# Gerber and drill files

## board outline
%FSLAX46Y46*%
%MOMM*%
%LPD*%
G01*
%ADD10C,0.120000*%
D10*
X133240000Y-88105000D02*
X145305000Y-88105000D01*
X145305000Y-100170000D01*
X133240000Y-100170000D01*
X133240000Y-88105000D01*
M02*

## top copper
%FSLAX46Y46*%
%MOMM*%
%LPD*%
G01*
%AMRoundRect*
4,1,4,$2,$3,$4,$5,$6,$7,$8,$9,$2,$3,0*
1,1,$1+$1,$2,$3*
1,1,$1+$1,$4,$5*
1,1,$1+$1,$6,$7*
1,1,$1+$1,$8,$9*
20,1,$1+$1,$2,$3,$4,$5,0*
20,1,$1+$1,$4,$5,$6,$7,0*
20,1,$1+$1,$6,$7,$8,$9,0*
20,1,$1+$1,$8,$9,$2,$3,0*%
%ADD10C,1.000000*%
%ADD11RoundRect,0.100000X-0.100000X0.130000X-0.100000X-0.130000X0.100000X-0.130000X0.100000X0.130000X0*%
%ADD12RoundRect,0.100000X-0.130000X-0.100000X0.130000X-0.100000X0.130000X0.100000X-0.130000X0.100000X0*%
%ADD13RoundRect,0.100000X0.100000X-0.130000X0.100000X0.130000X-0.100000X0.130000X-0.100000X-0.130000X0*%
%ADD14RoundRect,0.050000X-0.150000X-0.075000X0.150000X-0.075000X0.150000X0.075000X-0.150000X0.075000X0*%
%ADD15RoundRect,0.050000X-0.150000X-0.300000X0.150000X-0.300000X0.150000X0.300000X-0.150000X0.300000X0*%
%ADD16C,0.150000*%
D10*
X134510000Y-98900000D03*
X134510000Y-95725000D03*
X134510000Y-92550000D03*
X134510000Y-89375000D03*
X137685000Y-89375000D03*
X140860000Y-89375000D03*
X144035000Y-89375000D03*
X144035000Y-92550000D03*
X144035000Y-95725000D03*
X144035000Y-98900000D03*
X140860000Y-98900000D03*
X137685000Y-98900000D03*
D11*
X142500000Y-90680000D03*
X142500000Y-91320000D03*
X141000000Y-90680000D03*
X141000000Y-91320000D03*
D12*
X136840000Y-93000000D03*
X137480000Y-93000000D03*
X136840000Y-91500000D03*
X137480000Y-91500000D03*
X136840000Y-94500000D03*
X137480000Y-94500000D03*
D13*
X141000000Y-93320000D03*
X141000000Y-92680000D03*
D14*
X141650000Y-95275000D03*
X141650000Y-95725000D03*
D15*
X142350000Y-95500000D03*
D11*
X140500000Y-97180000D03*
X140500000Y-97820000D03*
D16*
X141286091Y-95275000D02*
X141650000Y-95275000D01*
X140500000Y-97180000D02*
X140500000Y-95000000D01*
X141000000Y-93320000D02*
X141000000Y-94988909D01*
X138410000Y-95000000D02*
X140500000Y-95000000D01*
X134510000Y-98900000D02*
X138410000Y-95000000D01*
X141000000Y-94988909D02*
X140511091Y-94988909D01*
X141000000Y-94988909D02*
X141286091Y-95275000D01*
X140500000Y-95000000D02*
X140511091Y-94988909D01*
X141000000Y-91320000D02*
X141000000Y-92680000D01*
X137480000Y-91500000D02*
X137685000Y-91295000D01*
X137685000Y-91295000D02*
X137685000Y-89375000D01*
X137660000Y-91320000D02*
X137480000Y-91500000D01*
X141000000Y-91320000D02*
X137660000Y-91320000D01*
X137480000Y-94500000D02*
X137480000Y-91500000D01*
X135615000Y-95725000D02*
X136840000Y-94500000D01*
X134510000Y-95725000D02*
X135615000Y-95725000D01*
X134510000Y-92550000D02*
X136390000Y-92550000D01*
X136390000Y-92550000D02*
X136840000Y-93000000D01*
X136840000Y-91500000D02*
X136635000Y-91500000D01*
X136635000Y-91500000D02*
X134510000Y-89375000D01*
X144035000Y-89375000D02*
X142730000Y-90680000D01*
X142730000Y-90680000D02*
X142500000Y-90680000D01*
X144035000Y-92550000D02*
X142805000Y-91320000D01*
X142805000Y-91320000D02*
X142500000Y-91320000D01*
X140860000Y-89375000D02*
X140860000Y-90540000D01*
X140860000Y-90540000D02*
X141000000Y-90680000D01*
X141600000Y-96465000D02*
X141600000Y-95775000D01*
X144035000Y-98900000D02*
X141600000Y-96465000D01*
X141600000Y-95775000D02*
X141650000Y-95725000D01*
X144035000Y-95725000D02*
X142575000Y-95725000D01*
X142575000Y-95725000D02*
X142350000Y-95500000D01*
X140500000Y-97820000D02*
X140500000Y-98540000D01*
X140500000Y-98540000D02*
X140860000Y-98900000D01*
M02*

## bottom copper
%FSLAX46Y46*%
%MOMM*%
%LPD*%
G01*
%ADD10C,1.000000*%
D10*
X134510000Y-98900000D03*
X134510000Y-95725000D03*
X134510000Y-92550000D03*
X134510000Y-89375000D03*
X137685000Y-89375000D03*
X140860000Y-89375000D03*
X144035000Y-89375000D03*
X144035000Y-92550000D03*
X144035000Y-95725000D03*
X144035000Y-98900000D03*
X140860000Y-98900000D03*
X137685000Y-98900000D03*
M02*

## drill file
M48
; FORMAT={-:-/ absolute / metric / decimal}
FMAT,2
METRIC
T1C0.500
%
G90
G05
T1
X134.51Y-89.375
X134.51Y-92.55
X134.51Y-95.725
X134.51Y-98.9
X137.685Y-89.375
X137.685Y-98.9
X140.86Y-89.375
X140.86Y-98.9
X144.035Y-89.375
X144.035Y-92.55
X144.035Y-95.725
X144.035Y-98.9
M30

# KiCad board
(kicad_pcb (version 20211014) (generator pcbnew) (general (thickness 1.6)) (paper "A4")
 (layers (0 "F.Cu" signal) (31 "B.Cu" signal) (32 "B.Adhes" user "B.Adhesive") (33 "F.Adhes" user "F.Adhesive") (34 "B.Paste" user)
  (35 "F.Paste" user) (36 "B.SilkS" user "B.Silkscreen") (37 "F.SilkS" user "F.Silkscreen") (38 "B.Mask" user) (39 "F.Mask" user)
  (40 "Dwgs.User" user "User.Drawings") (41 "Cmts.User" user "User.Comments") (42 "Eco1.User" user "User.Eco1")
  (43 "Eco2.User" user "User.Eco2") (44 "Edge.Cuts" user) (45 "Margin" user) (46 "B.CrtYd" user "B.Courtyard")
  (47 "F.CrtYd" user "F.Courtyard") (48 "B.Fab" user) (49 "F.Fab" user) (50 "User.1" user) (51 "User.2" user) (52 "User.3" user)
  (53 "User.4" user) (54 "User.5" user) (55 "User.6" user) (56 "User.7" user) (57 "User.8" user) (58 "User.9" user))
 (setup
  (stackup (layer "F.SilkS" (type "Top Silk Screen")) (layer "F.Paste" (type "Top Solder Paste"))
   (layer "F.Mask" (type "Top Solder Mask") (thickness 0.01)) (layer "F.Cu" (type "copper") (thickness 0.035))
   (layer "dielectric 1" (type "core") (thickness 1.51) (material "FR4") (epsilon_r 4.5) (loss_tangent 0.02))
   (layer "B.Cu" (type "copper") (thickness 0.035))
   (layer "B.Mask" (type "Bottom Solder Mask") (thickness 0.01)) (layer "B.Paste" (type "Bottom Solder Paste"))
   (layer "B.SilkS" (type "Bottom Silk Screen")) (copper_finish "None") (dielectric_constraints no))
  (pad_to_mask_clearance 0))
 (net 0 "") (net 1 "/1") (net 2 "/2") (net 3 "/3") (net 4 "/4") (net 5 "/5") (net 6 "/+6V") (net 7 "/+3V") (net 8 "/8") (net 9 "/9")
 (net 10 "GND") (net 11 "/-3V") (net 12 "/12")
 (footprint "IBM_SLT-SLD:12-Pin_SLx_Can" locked (layer "F.Cu") (at 134.51 98.9)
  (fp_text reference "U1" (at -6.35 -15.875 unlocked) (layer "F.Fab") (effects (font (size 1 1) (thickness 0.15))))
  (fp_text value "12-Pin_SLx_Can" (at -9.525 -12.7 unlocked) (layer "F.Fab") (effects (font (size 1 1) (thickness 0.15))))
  (fp_rect (start -1.27 -10.795) (end 10.795 1.27) (layer "Edge.Cuts") (width 0.12) (fill none))
  (pad "1" thru_hole circle locked (at 0 0) (size 1 1) (drill 0.5) (layers *.Cu *.Mask) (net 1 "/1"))
  (pad "2" thru_hole circle locked (at 0 -3.175) (size 1 1) (drill 0.5) (layers *.Cu *.Mask) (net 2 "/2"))
  (pad "3" thru_hole circle locked (at 0 -6.35) (size 1 1) (drill 0.5) (layers *.Cu *.Mask) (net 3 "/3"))
  (pad "4" thru_hole circle locked (at 0 -9.525) (size 1 1) (drill 0.5) (layers *.Cu *.Mask) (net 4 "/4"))
  (pad "5" thru_hole circle locked (at 3.175 -9.525) (size 1 1) (drill 0.5) (layers *.Cu *.Mask) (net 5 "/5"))
  (pad "6" thru_hole circle locked (at 6.35 -9.525) (size 1 1) (drill 0.5) (layers *.Cu *.Mask) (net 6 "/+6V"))
  (pad "7" thru_hole circle locked (at 9.525 -9.525) (size 1 1) (drill 0.5) (layers *.Cu *.Mask) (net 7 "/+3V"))
  (pad "8" thru_hole circle locked (at 9.525 -6.35) (size 1 1) (drill 0.5) (layers *.Cu *.Mask) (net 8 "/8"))
  (pad "9" thru_hole circle locked (at 9.525 -3.175) (size 1 1) (drill 0.5) (layers *.Cu *.Mask) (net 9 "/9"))
  (pad "10" thru_hole circle locked (at 9.525 0) (size 1 1) (drill 0.5) (layers *.Cu *.Mask) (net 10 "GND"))
  (pad "11" thru_hole circle locked (at 6.35 0) (size 1 1) (drill 0.5) (layers *.Cu *.Mask) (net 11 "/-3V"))
  (pad "12" thru_hole circle locked (at 3.175 0) (size 1 1) (drill 0.5) (layers *.Cu *.Mask) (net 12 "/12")))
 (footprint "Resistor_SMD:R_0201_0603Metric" (layer "F.Cu") (at 142.5 91 -90)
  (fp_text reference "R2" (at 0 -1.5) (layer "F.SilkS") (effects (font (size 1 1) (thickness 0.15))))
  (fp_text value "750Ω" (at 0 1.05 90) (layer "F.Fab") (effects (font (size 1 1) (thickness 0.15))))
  (pad "" smd roundrect (at 0.345 0 270) (size 0.318 0.36) (layers "F.Paste") (roundrect_rratio 0.25))
  (pad "" smd roundrect (at -0.345 0 270) (size 0.318 0.36) (layers "F.Paste") (roundrect_rratio 0.25))
  (pad "1" smd roundrect (at -0.32 0 270) (size 0.46 0.4) (layers "F.Cu" "F.Mask") (roundrect_rratio 0.25) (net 7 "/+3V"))
  (pad "2" smd roundrect (at 0.32 0 270) (size 0.46 0.4) (layers "F.Cu" "F.Mask") (roundrect_rratio 0.25) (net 8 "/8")))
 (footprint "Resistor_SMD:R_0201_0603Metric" (layer "F.Cu") (at 141 91 -90)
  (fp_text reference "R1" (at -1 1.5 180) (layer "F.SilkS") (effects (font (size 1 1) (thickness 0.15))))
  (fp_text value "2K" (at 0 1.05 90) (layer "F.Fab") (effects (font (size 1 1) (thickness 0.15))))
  (pad "" smd roundrect (at 0.345 0 270) (size 0.318 0.36) (layers "F.Paste") (roundrect_rratio 0.25))
  (pad "" smd roundrect (at -0.345 0 270) (size 0.318 0.36) (layers "F.Paste") (roundrect_rratio 0.25))
  (pad "1" smd roundrect (at -0.32 0 270) (size 0.46 0.4) (layers "F.Cu" "F.Mask") (roundrect_rratio 0.25) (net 6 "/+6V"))
  (pad "2" smd roundrect (at 0.32 0 270) (size 0.46 0.4) (layers "F.Cu" "F.Mask") (roundrect_rratio 0.25) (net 5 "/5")))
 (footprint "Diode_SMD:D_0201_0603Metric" (layer "F.Cu") (at 137.16 93)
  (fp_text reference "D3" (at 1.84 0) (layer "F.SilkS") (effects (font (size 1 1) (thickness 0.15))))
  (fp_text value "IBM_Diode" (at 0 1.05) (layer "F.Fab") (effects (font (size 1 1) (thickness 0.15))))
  (pad "" smd roundrect (at 0.345 0) (size 0.318 0.36) (layers "F.Paste") (roundrect_rratio 0.25))
  (pad "" smd roundrect (at -0.345 0) (size 0.318 0.36) (layers "F.Paste") (roundrect_rratio 0.25))
  (pad "1" smd roundrect (at -0.32 0) (size 0.46 0.4) (layers "F.Cu" "F.Mask") (roundrect_rratio 0.25) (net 3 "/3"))
  (pad "2" smd roundrect (at 0.32 0) (size 0.46 0.4) (layers "F.Cu" "F.Mask") (roundrect_rratio 0.25) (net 5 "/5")))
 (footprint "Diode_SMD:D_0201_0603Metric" (layer "F.Cu") (at 137.16 91.5)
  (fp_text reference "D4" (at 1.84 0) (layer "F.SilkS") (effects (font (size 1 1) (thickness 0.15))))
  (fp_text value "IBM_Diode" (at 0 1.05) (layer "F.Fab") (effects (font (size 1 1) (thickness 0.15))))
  (pad "" smd roundrect (at 0.345 0) (size 0.318 0.36) (layers "F.Paste") (roundrect_rratio 0.25))
  (pad "" smd roundrect (at -0.345 0) (size 0.318 0.36) (layers "F.Paste") (roundrect_rratio 0.25))
  (pad "1" smd roundrect (at -0.32 0) (size 0.46 0.4) (layers "F.Cu" "F.Mask") (roundrect_rratio 0.25) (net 4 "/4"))
  (pad "2" smd roundrect (at 0.32 0) (size 0.46 0.4) (layers "F.Cu" "F.Mask") (roundrect_rratio 0.25) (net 5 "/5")))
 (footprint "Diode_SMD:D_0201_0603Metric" (layer "F.Cu") (at 137.16 94.5)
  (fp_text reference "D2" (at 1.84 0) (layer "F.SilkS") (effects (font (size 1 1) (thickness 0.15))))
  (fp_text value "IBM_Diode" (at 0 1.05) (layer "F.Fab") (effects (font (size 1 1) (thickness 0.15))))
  (pad "" smd roundrect (at -0.345 0) (size 0.318 0.36) (layers "F.Paste") (roundrect_rratio 0.25))
  (pad "" smd roundrect (at 0.345 0) (size 0.318 0.36) (layers "F.Paste") (roundrect_rratio 0.25))
  (pad "1" smd roundrect (at -0.32 0) (size 0.46 0.4) (layers "F.Cu" "F.Mask") (roundrect_rratio 0.25) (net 2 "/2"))
  (pad "2" smd roundrect (at 0.32 0) (size 0.46 0.4) (layers "F.Cu" "F.Mask") (roundrect_rratio 0.25) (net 5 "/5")))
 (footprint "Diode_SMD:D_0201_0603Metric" (layer "F.Cu") (at 141 93 90)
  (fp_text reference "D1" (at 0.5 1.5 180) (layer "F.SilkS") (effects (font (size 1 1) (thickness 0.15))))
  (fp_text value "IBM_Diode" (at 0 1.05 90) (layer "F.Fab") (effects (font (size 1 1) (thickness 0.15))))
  (pad "" smd roundrect (at -0.345 0 90) (size 0.318 0.36) (layers "F.Paste") (roundrect_rratio 0.25))
  (pad "" smd roundrect (at 0.345 0 90) (size 0.318 0.36) (layers "F.Paste") (roundrect_rratio 0.25))
  (pad "1" smd roundrect (at -0.32 0 90) (size 0.46 0.4) (layers "F.Cu" "F.Mask") (roundrect_rratio 0.25) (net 1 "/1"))
  (pad "2" smd roundrect (at 0.32 0 90) (size 0.46 0.4) (layers "F.Cu" "F.Mask") (roundrect_rratio 0.25) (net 5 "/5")))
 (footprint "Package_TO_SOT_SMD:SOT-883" (layer "F.Cu") (at 142 95.5)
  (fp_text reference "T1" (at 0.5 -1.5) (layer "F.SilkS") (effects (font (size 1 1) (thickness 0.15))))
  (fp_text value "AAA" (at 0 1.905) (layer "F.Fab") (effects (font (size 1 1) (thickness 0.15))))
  (pad "1" smd roundrect (at -0.35 -0.225) (size 0.4 0.25) (layers "F.Cu" "F.Paste" "F.Mask") (roundrect_rratio 0.2) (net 1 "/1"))
  (pad "2" smd roundrect (at -0.35 0.225) (size 0.4 0.25) (layers "F.Cu" "F.Paste" "F.Mask") (roundrect_rratio 0.2) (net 10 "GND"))
  (pad "3" smd roundrect (at 0.35 0) (size 0.4 0.7) (layers "F.Cu" "F.Paste" "F.Mask") (roundrect_rratio 0.125) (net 9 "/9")))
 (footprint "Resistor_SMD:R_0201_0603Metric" (layer "F.Cu") (at 140.5 97.5 -90)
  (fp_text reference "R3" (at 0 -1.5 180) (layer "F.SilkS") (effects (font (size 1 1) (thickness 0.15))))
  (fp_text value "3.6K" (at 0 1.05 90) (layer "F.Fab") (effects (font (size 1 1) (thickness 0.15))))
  (pad "" smd roundrect (at -0.345 0 270) (size 0.318 0.36) (layers "F.Paste") (roundrect_rratio 0.25))
  (pad "" smd roundrect (at 0.345 0 270) (size 0.318 0.36) (layers "F.Paste") (roundrect_rratio 0.25))
  (pad "1" smd roundrect (at -0.32 0 270) (size 0.46 0.4) (layers "F.Cu" "F.Mask") (roundrect_rratio 0.25) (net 1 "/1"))
  (pad "2" smd roundrect (at 0.32 0 270) (size 0.46 0.4) (layers "F.Cu" "F.Mask") (roundrect_rratio 0.25) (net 11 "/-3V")))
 (segment (start 141.286091 95.275) (end 141.65 95.275) (width 0.15) (layer "F.Cu") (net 1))
 (segment (start 140.5 97.18) (end 140.5 95) (width 0.15) (layer "F.Cu") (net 1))
 (segment (start 141 93.32) (end 141 94.988909) (width 0.15) (layer "F.Cu") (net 1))
 (segment (start 138.41 95) (end 140.5 95) (width 0.15) (layer "F.Cu") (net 1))
 (segment (start 134.51 98.9) (end 138.41 95) (width 0.15) (layer "F.Cu") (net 1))
 (segment (start 141 94.988909) (end 140.511091 94.988909) (width 0.15) (layer "F.Cu") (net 1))
 (segment (start 141 94.988909) (end 141.286091 95.275) (width 0.15) (layer "F.Cu") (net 1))
 (segment (start 140.5 95) (end 140.511091 94.988909) (width 0.15) (layer "F.Cu") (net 1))
 (segment (start 141 91.32) (end 141 92.68) (width 0.15) (layer "F.Cu") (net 5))
 (segment (start 137.48 91.5) (end 137.685 91.295) (width 0.15) (layer "F.Cu") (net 5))
 (segment (start 137.685 91.295) (end 137.685 89.375) (width 0.15) (layer "F.Cu") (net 5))
 (segment (start 137.66 91.32) (end 137.48 91.5) (width 0.15) (layer "F.Cu") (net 5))
 (segment (start 141 91.32) (end 137.66 91.32) (width 0.15) (layer "F.Cu") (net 5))
 (segment (start 137.48 94.5) (end 137.48 91.5) (width 0.15) (layer "F.Cu") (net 5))
 (segment (start 135.615 95.725) (end 136.84 94.5) (width 0.15) (layer "F.Cu") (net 2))
 (segment (start 134.51 95.725) (end 135.615 95.725) (width 0.15) (layer "F.Cu") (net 2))
 (segment (start 134.51 92.55) (end 136.39 92.55) (width 0.15) (layer "F.Cu") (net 3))
 (segment (start 136.39 92.55) (end 136.84 93) (width 0.15) (layer "F.Cu") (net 3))
 (segment (start 136.84 91.5) (end 136.635 91.5) (width 0.15) (layer "F.Cu") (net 4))
 (segment (start 136.635 91.5) (end 134.51 89.375) (width 0.15) (layer "F.Cu") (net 4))
 (segment (start 144.035 89.375) (end 142.73 90.68) (width 0.15) (layer "F.Cu") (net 7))
 (segment (start 142.73 90.68) (end 142.5 90.68) (width 0.15) (layer "F.Cu") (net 7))
 (segment (start 144.035 92.55) (end 142.805 91.32) (width 0.15) (layer "F.Cu") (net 8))
 (segment (start 142.805 91.32) (end 142.5 91.32) (width 0.15) (layer "F.Cu") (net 8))
 (segment (start 140.86 89.375) (end 140.86 90.54) (width 0.15) (layer "F.Cu") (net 6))
 (segment (start 140.86 90.54) (end 141 90.68) (width 0.15) (layer "F.Cu") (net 6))
 (segment (start 141.6 96.465) (end 141.6 95.775) (width 0.15) (layer "F.Cu") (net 10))
 (segment (start 144.035 98.9) (end 141.6 96.465) (width 0.15) (layer "F.Cu") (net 10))
 (segment (start 141.6 95.775) (end 141.65 95.725) (width 0.15) (layer "F.Cu") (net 10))
 (segment (start 144.035 95.725) (end 142.575 95.725) (width 0.15) (layer "F.Cu") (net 9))
 (segment (start 142.575 95.725) (end 142.35 95.5) (width 0.15) (layer "F.Cu") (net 9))
 (segment (start 140.5 97.82) (end 140.5 98.54) (width 0.15) (layer "F.Cu") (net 11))
 (segment (start 140.5 98.54) (end 140.86 98.9) (width 0.15) (layer "F.Cu") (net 11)))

